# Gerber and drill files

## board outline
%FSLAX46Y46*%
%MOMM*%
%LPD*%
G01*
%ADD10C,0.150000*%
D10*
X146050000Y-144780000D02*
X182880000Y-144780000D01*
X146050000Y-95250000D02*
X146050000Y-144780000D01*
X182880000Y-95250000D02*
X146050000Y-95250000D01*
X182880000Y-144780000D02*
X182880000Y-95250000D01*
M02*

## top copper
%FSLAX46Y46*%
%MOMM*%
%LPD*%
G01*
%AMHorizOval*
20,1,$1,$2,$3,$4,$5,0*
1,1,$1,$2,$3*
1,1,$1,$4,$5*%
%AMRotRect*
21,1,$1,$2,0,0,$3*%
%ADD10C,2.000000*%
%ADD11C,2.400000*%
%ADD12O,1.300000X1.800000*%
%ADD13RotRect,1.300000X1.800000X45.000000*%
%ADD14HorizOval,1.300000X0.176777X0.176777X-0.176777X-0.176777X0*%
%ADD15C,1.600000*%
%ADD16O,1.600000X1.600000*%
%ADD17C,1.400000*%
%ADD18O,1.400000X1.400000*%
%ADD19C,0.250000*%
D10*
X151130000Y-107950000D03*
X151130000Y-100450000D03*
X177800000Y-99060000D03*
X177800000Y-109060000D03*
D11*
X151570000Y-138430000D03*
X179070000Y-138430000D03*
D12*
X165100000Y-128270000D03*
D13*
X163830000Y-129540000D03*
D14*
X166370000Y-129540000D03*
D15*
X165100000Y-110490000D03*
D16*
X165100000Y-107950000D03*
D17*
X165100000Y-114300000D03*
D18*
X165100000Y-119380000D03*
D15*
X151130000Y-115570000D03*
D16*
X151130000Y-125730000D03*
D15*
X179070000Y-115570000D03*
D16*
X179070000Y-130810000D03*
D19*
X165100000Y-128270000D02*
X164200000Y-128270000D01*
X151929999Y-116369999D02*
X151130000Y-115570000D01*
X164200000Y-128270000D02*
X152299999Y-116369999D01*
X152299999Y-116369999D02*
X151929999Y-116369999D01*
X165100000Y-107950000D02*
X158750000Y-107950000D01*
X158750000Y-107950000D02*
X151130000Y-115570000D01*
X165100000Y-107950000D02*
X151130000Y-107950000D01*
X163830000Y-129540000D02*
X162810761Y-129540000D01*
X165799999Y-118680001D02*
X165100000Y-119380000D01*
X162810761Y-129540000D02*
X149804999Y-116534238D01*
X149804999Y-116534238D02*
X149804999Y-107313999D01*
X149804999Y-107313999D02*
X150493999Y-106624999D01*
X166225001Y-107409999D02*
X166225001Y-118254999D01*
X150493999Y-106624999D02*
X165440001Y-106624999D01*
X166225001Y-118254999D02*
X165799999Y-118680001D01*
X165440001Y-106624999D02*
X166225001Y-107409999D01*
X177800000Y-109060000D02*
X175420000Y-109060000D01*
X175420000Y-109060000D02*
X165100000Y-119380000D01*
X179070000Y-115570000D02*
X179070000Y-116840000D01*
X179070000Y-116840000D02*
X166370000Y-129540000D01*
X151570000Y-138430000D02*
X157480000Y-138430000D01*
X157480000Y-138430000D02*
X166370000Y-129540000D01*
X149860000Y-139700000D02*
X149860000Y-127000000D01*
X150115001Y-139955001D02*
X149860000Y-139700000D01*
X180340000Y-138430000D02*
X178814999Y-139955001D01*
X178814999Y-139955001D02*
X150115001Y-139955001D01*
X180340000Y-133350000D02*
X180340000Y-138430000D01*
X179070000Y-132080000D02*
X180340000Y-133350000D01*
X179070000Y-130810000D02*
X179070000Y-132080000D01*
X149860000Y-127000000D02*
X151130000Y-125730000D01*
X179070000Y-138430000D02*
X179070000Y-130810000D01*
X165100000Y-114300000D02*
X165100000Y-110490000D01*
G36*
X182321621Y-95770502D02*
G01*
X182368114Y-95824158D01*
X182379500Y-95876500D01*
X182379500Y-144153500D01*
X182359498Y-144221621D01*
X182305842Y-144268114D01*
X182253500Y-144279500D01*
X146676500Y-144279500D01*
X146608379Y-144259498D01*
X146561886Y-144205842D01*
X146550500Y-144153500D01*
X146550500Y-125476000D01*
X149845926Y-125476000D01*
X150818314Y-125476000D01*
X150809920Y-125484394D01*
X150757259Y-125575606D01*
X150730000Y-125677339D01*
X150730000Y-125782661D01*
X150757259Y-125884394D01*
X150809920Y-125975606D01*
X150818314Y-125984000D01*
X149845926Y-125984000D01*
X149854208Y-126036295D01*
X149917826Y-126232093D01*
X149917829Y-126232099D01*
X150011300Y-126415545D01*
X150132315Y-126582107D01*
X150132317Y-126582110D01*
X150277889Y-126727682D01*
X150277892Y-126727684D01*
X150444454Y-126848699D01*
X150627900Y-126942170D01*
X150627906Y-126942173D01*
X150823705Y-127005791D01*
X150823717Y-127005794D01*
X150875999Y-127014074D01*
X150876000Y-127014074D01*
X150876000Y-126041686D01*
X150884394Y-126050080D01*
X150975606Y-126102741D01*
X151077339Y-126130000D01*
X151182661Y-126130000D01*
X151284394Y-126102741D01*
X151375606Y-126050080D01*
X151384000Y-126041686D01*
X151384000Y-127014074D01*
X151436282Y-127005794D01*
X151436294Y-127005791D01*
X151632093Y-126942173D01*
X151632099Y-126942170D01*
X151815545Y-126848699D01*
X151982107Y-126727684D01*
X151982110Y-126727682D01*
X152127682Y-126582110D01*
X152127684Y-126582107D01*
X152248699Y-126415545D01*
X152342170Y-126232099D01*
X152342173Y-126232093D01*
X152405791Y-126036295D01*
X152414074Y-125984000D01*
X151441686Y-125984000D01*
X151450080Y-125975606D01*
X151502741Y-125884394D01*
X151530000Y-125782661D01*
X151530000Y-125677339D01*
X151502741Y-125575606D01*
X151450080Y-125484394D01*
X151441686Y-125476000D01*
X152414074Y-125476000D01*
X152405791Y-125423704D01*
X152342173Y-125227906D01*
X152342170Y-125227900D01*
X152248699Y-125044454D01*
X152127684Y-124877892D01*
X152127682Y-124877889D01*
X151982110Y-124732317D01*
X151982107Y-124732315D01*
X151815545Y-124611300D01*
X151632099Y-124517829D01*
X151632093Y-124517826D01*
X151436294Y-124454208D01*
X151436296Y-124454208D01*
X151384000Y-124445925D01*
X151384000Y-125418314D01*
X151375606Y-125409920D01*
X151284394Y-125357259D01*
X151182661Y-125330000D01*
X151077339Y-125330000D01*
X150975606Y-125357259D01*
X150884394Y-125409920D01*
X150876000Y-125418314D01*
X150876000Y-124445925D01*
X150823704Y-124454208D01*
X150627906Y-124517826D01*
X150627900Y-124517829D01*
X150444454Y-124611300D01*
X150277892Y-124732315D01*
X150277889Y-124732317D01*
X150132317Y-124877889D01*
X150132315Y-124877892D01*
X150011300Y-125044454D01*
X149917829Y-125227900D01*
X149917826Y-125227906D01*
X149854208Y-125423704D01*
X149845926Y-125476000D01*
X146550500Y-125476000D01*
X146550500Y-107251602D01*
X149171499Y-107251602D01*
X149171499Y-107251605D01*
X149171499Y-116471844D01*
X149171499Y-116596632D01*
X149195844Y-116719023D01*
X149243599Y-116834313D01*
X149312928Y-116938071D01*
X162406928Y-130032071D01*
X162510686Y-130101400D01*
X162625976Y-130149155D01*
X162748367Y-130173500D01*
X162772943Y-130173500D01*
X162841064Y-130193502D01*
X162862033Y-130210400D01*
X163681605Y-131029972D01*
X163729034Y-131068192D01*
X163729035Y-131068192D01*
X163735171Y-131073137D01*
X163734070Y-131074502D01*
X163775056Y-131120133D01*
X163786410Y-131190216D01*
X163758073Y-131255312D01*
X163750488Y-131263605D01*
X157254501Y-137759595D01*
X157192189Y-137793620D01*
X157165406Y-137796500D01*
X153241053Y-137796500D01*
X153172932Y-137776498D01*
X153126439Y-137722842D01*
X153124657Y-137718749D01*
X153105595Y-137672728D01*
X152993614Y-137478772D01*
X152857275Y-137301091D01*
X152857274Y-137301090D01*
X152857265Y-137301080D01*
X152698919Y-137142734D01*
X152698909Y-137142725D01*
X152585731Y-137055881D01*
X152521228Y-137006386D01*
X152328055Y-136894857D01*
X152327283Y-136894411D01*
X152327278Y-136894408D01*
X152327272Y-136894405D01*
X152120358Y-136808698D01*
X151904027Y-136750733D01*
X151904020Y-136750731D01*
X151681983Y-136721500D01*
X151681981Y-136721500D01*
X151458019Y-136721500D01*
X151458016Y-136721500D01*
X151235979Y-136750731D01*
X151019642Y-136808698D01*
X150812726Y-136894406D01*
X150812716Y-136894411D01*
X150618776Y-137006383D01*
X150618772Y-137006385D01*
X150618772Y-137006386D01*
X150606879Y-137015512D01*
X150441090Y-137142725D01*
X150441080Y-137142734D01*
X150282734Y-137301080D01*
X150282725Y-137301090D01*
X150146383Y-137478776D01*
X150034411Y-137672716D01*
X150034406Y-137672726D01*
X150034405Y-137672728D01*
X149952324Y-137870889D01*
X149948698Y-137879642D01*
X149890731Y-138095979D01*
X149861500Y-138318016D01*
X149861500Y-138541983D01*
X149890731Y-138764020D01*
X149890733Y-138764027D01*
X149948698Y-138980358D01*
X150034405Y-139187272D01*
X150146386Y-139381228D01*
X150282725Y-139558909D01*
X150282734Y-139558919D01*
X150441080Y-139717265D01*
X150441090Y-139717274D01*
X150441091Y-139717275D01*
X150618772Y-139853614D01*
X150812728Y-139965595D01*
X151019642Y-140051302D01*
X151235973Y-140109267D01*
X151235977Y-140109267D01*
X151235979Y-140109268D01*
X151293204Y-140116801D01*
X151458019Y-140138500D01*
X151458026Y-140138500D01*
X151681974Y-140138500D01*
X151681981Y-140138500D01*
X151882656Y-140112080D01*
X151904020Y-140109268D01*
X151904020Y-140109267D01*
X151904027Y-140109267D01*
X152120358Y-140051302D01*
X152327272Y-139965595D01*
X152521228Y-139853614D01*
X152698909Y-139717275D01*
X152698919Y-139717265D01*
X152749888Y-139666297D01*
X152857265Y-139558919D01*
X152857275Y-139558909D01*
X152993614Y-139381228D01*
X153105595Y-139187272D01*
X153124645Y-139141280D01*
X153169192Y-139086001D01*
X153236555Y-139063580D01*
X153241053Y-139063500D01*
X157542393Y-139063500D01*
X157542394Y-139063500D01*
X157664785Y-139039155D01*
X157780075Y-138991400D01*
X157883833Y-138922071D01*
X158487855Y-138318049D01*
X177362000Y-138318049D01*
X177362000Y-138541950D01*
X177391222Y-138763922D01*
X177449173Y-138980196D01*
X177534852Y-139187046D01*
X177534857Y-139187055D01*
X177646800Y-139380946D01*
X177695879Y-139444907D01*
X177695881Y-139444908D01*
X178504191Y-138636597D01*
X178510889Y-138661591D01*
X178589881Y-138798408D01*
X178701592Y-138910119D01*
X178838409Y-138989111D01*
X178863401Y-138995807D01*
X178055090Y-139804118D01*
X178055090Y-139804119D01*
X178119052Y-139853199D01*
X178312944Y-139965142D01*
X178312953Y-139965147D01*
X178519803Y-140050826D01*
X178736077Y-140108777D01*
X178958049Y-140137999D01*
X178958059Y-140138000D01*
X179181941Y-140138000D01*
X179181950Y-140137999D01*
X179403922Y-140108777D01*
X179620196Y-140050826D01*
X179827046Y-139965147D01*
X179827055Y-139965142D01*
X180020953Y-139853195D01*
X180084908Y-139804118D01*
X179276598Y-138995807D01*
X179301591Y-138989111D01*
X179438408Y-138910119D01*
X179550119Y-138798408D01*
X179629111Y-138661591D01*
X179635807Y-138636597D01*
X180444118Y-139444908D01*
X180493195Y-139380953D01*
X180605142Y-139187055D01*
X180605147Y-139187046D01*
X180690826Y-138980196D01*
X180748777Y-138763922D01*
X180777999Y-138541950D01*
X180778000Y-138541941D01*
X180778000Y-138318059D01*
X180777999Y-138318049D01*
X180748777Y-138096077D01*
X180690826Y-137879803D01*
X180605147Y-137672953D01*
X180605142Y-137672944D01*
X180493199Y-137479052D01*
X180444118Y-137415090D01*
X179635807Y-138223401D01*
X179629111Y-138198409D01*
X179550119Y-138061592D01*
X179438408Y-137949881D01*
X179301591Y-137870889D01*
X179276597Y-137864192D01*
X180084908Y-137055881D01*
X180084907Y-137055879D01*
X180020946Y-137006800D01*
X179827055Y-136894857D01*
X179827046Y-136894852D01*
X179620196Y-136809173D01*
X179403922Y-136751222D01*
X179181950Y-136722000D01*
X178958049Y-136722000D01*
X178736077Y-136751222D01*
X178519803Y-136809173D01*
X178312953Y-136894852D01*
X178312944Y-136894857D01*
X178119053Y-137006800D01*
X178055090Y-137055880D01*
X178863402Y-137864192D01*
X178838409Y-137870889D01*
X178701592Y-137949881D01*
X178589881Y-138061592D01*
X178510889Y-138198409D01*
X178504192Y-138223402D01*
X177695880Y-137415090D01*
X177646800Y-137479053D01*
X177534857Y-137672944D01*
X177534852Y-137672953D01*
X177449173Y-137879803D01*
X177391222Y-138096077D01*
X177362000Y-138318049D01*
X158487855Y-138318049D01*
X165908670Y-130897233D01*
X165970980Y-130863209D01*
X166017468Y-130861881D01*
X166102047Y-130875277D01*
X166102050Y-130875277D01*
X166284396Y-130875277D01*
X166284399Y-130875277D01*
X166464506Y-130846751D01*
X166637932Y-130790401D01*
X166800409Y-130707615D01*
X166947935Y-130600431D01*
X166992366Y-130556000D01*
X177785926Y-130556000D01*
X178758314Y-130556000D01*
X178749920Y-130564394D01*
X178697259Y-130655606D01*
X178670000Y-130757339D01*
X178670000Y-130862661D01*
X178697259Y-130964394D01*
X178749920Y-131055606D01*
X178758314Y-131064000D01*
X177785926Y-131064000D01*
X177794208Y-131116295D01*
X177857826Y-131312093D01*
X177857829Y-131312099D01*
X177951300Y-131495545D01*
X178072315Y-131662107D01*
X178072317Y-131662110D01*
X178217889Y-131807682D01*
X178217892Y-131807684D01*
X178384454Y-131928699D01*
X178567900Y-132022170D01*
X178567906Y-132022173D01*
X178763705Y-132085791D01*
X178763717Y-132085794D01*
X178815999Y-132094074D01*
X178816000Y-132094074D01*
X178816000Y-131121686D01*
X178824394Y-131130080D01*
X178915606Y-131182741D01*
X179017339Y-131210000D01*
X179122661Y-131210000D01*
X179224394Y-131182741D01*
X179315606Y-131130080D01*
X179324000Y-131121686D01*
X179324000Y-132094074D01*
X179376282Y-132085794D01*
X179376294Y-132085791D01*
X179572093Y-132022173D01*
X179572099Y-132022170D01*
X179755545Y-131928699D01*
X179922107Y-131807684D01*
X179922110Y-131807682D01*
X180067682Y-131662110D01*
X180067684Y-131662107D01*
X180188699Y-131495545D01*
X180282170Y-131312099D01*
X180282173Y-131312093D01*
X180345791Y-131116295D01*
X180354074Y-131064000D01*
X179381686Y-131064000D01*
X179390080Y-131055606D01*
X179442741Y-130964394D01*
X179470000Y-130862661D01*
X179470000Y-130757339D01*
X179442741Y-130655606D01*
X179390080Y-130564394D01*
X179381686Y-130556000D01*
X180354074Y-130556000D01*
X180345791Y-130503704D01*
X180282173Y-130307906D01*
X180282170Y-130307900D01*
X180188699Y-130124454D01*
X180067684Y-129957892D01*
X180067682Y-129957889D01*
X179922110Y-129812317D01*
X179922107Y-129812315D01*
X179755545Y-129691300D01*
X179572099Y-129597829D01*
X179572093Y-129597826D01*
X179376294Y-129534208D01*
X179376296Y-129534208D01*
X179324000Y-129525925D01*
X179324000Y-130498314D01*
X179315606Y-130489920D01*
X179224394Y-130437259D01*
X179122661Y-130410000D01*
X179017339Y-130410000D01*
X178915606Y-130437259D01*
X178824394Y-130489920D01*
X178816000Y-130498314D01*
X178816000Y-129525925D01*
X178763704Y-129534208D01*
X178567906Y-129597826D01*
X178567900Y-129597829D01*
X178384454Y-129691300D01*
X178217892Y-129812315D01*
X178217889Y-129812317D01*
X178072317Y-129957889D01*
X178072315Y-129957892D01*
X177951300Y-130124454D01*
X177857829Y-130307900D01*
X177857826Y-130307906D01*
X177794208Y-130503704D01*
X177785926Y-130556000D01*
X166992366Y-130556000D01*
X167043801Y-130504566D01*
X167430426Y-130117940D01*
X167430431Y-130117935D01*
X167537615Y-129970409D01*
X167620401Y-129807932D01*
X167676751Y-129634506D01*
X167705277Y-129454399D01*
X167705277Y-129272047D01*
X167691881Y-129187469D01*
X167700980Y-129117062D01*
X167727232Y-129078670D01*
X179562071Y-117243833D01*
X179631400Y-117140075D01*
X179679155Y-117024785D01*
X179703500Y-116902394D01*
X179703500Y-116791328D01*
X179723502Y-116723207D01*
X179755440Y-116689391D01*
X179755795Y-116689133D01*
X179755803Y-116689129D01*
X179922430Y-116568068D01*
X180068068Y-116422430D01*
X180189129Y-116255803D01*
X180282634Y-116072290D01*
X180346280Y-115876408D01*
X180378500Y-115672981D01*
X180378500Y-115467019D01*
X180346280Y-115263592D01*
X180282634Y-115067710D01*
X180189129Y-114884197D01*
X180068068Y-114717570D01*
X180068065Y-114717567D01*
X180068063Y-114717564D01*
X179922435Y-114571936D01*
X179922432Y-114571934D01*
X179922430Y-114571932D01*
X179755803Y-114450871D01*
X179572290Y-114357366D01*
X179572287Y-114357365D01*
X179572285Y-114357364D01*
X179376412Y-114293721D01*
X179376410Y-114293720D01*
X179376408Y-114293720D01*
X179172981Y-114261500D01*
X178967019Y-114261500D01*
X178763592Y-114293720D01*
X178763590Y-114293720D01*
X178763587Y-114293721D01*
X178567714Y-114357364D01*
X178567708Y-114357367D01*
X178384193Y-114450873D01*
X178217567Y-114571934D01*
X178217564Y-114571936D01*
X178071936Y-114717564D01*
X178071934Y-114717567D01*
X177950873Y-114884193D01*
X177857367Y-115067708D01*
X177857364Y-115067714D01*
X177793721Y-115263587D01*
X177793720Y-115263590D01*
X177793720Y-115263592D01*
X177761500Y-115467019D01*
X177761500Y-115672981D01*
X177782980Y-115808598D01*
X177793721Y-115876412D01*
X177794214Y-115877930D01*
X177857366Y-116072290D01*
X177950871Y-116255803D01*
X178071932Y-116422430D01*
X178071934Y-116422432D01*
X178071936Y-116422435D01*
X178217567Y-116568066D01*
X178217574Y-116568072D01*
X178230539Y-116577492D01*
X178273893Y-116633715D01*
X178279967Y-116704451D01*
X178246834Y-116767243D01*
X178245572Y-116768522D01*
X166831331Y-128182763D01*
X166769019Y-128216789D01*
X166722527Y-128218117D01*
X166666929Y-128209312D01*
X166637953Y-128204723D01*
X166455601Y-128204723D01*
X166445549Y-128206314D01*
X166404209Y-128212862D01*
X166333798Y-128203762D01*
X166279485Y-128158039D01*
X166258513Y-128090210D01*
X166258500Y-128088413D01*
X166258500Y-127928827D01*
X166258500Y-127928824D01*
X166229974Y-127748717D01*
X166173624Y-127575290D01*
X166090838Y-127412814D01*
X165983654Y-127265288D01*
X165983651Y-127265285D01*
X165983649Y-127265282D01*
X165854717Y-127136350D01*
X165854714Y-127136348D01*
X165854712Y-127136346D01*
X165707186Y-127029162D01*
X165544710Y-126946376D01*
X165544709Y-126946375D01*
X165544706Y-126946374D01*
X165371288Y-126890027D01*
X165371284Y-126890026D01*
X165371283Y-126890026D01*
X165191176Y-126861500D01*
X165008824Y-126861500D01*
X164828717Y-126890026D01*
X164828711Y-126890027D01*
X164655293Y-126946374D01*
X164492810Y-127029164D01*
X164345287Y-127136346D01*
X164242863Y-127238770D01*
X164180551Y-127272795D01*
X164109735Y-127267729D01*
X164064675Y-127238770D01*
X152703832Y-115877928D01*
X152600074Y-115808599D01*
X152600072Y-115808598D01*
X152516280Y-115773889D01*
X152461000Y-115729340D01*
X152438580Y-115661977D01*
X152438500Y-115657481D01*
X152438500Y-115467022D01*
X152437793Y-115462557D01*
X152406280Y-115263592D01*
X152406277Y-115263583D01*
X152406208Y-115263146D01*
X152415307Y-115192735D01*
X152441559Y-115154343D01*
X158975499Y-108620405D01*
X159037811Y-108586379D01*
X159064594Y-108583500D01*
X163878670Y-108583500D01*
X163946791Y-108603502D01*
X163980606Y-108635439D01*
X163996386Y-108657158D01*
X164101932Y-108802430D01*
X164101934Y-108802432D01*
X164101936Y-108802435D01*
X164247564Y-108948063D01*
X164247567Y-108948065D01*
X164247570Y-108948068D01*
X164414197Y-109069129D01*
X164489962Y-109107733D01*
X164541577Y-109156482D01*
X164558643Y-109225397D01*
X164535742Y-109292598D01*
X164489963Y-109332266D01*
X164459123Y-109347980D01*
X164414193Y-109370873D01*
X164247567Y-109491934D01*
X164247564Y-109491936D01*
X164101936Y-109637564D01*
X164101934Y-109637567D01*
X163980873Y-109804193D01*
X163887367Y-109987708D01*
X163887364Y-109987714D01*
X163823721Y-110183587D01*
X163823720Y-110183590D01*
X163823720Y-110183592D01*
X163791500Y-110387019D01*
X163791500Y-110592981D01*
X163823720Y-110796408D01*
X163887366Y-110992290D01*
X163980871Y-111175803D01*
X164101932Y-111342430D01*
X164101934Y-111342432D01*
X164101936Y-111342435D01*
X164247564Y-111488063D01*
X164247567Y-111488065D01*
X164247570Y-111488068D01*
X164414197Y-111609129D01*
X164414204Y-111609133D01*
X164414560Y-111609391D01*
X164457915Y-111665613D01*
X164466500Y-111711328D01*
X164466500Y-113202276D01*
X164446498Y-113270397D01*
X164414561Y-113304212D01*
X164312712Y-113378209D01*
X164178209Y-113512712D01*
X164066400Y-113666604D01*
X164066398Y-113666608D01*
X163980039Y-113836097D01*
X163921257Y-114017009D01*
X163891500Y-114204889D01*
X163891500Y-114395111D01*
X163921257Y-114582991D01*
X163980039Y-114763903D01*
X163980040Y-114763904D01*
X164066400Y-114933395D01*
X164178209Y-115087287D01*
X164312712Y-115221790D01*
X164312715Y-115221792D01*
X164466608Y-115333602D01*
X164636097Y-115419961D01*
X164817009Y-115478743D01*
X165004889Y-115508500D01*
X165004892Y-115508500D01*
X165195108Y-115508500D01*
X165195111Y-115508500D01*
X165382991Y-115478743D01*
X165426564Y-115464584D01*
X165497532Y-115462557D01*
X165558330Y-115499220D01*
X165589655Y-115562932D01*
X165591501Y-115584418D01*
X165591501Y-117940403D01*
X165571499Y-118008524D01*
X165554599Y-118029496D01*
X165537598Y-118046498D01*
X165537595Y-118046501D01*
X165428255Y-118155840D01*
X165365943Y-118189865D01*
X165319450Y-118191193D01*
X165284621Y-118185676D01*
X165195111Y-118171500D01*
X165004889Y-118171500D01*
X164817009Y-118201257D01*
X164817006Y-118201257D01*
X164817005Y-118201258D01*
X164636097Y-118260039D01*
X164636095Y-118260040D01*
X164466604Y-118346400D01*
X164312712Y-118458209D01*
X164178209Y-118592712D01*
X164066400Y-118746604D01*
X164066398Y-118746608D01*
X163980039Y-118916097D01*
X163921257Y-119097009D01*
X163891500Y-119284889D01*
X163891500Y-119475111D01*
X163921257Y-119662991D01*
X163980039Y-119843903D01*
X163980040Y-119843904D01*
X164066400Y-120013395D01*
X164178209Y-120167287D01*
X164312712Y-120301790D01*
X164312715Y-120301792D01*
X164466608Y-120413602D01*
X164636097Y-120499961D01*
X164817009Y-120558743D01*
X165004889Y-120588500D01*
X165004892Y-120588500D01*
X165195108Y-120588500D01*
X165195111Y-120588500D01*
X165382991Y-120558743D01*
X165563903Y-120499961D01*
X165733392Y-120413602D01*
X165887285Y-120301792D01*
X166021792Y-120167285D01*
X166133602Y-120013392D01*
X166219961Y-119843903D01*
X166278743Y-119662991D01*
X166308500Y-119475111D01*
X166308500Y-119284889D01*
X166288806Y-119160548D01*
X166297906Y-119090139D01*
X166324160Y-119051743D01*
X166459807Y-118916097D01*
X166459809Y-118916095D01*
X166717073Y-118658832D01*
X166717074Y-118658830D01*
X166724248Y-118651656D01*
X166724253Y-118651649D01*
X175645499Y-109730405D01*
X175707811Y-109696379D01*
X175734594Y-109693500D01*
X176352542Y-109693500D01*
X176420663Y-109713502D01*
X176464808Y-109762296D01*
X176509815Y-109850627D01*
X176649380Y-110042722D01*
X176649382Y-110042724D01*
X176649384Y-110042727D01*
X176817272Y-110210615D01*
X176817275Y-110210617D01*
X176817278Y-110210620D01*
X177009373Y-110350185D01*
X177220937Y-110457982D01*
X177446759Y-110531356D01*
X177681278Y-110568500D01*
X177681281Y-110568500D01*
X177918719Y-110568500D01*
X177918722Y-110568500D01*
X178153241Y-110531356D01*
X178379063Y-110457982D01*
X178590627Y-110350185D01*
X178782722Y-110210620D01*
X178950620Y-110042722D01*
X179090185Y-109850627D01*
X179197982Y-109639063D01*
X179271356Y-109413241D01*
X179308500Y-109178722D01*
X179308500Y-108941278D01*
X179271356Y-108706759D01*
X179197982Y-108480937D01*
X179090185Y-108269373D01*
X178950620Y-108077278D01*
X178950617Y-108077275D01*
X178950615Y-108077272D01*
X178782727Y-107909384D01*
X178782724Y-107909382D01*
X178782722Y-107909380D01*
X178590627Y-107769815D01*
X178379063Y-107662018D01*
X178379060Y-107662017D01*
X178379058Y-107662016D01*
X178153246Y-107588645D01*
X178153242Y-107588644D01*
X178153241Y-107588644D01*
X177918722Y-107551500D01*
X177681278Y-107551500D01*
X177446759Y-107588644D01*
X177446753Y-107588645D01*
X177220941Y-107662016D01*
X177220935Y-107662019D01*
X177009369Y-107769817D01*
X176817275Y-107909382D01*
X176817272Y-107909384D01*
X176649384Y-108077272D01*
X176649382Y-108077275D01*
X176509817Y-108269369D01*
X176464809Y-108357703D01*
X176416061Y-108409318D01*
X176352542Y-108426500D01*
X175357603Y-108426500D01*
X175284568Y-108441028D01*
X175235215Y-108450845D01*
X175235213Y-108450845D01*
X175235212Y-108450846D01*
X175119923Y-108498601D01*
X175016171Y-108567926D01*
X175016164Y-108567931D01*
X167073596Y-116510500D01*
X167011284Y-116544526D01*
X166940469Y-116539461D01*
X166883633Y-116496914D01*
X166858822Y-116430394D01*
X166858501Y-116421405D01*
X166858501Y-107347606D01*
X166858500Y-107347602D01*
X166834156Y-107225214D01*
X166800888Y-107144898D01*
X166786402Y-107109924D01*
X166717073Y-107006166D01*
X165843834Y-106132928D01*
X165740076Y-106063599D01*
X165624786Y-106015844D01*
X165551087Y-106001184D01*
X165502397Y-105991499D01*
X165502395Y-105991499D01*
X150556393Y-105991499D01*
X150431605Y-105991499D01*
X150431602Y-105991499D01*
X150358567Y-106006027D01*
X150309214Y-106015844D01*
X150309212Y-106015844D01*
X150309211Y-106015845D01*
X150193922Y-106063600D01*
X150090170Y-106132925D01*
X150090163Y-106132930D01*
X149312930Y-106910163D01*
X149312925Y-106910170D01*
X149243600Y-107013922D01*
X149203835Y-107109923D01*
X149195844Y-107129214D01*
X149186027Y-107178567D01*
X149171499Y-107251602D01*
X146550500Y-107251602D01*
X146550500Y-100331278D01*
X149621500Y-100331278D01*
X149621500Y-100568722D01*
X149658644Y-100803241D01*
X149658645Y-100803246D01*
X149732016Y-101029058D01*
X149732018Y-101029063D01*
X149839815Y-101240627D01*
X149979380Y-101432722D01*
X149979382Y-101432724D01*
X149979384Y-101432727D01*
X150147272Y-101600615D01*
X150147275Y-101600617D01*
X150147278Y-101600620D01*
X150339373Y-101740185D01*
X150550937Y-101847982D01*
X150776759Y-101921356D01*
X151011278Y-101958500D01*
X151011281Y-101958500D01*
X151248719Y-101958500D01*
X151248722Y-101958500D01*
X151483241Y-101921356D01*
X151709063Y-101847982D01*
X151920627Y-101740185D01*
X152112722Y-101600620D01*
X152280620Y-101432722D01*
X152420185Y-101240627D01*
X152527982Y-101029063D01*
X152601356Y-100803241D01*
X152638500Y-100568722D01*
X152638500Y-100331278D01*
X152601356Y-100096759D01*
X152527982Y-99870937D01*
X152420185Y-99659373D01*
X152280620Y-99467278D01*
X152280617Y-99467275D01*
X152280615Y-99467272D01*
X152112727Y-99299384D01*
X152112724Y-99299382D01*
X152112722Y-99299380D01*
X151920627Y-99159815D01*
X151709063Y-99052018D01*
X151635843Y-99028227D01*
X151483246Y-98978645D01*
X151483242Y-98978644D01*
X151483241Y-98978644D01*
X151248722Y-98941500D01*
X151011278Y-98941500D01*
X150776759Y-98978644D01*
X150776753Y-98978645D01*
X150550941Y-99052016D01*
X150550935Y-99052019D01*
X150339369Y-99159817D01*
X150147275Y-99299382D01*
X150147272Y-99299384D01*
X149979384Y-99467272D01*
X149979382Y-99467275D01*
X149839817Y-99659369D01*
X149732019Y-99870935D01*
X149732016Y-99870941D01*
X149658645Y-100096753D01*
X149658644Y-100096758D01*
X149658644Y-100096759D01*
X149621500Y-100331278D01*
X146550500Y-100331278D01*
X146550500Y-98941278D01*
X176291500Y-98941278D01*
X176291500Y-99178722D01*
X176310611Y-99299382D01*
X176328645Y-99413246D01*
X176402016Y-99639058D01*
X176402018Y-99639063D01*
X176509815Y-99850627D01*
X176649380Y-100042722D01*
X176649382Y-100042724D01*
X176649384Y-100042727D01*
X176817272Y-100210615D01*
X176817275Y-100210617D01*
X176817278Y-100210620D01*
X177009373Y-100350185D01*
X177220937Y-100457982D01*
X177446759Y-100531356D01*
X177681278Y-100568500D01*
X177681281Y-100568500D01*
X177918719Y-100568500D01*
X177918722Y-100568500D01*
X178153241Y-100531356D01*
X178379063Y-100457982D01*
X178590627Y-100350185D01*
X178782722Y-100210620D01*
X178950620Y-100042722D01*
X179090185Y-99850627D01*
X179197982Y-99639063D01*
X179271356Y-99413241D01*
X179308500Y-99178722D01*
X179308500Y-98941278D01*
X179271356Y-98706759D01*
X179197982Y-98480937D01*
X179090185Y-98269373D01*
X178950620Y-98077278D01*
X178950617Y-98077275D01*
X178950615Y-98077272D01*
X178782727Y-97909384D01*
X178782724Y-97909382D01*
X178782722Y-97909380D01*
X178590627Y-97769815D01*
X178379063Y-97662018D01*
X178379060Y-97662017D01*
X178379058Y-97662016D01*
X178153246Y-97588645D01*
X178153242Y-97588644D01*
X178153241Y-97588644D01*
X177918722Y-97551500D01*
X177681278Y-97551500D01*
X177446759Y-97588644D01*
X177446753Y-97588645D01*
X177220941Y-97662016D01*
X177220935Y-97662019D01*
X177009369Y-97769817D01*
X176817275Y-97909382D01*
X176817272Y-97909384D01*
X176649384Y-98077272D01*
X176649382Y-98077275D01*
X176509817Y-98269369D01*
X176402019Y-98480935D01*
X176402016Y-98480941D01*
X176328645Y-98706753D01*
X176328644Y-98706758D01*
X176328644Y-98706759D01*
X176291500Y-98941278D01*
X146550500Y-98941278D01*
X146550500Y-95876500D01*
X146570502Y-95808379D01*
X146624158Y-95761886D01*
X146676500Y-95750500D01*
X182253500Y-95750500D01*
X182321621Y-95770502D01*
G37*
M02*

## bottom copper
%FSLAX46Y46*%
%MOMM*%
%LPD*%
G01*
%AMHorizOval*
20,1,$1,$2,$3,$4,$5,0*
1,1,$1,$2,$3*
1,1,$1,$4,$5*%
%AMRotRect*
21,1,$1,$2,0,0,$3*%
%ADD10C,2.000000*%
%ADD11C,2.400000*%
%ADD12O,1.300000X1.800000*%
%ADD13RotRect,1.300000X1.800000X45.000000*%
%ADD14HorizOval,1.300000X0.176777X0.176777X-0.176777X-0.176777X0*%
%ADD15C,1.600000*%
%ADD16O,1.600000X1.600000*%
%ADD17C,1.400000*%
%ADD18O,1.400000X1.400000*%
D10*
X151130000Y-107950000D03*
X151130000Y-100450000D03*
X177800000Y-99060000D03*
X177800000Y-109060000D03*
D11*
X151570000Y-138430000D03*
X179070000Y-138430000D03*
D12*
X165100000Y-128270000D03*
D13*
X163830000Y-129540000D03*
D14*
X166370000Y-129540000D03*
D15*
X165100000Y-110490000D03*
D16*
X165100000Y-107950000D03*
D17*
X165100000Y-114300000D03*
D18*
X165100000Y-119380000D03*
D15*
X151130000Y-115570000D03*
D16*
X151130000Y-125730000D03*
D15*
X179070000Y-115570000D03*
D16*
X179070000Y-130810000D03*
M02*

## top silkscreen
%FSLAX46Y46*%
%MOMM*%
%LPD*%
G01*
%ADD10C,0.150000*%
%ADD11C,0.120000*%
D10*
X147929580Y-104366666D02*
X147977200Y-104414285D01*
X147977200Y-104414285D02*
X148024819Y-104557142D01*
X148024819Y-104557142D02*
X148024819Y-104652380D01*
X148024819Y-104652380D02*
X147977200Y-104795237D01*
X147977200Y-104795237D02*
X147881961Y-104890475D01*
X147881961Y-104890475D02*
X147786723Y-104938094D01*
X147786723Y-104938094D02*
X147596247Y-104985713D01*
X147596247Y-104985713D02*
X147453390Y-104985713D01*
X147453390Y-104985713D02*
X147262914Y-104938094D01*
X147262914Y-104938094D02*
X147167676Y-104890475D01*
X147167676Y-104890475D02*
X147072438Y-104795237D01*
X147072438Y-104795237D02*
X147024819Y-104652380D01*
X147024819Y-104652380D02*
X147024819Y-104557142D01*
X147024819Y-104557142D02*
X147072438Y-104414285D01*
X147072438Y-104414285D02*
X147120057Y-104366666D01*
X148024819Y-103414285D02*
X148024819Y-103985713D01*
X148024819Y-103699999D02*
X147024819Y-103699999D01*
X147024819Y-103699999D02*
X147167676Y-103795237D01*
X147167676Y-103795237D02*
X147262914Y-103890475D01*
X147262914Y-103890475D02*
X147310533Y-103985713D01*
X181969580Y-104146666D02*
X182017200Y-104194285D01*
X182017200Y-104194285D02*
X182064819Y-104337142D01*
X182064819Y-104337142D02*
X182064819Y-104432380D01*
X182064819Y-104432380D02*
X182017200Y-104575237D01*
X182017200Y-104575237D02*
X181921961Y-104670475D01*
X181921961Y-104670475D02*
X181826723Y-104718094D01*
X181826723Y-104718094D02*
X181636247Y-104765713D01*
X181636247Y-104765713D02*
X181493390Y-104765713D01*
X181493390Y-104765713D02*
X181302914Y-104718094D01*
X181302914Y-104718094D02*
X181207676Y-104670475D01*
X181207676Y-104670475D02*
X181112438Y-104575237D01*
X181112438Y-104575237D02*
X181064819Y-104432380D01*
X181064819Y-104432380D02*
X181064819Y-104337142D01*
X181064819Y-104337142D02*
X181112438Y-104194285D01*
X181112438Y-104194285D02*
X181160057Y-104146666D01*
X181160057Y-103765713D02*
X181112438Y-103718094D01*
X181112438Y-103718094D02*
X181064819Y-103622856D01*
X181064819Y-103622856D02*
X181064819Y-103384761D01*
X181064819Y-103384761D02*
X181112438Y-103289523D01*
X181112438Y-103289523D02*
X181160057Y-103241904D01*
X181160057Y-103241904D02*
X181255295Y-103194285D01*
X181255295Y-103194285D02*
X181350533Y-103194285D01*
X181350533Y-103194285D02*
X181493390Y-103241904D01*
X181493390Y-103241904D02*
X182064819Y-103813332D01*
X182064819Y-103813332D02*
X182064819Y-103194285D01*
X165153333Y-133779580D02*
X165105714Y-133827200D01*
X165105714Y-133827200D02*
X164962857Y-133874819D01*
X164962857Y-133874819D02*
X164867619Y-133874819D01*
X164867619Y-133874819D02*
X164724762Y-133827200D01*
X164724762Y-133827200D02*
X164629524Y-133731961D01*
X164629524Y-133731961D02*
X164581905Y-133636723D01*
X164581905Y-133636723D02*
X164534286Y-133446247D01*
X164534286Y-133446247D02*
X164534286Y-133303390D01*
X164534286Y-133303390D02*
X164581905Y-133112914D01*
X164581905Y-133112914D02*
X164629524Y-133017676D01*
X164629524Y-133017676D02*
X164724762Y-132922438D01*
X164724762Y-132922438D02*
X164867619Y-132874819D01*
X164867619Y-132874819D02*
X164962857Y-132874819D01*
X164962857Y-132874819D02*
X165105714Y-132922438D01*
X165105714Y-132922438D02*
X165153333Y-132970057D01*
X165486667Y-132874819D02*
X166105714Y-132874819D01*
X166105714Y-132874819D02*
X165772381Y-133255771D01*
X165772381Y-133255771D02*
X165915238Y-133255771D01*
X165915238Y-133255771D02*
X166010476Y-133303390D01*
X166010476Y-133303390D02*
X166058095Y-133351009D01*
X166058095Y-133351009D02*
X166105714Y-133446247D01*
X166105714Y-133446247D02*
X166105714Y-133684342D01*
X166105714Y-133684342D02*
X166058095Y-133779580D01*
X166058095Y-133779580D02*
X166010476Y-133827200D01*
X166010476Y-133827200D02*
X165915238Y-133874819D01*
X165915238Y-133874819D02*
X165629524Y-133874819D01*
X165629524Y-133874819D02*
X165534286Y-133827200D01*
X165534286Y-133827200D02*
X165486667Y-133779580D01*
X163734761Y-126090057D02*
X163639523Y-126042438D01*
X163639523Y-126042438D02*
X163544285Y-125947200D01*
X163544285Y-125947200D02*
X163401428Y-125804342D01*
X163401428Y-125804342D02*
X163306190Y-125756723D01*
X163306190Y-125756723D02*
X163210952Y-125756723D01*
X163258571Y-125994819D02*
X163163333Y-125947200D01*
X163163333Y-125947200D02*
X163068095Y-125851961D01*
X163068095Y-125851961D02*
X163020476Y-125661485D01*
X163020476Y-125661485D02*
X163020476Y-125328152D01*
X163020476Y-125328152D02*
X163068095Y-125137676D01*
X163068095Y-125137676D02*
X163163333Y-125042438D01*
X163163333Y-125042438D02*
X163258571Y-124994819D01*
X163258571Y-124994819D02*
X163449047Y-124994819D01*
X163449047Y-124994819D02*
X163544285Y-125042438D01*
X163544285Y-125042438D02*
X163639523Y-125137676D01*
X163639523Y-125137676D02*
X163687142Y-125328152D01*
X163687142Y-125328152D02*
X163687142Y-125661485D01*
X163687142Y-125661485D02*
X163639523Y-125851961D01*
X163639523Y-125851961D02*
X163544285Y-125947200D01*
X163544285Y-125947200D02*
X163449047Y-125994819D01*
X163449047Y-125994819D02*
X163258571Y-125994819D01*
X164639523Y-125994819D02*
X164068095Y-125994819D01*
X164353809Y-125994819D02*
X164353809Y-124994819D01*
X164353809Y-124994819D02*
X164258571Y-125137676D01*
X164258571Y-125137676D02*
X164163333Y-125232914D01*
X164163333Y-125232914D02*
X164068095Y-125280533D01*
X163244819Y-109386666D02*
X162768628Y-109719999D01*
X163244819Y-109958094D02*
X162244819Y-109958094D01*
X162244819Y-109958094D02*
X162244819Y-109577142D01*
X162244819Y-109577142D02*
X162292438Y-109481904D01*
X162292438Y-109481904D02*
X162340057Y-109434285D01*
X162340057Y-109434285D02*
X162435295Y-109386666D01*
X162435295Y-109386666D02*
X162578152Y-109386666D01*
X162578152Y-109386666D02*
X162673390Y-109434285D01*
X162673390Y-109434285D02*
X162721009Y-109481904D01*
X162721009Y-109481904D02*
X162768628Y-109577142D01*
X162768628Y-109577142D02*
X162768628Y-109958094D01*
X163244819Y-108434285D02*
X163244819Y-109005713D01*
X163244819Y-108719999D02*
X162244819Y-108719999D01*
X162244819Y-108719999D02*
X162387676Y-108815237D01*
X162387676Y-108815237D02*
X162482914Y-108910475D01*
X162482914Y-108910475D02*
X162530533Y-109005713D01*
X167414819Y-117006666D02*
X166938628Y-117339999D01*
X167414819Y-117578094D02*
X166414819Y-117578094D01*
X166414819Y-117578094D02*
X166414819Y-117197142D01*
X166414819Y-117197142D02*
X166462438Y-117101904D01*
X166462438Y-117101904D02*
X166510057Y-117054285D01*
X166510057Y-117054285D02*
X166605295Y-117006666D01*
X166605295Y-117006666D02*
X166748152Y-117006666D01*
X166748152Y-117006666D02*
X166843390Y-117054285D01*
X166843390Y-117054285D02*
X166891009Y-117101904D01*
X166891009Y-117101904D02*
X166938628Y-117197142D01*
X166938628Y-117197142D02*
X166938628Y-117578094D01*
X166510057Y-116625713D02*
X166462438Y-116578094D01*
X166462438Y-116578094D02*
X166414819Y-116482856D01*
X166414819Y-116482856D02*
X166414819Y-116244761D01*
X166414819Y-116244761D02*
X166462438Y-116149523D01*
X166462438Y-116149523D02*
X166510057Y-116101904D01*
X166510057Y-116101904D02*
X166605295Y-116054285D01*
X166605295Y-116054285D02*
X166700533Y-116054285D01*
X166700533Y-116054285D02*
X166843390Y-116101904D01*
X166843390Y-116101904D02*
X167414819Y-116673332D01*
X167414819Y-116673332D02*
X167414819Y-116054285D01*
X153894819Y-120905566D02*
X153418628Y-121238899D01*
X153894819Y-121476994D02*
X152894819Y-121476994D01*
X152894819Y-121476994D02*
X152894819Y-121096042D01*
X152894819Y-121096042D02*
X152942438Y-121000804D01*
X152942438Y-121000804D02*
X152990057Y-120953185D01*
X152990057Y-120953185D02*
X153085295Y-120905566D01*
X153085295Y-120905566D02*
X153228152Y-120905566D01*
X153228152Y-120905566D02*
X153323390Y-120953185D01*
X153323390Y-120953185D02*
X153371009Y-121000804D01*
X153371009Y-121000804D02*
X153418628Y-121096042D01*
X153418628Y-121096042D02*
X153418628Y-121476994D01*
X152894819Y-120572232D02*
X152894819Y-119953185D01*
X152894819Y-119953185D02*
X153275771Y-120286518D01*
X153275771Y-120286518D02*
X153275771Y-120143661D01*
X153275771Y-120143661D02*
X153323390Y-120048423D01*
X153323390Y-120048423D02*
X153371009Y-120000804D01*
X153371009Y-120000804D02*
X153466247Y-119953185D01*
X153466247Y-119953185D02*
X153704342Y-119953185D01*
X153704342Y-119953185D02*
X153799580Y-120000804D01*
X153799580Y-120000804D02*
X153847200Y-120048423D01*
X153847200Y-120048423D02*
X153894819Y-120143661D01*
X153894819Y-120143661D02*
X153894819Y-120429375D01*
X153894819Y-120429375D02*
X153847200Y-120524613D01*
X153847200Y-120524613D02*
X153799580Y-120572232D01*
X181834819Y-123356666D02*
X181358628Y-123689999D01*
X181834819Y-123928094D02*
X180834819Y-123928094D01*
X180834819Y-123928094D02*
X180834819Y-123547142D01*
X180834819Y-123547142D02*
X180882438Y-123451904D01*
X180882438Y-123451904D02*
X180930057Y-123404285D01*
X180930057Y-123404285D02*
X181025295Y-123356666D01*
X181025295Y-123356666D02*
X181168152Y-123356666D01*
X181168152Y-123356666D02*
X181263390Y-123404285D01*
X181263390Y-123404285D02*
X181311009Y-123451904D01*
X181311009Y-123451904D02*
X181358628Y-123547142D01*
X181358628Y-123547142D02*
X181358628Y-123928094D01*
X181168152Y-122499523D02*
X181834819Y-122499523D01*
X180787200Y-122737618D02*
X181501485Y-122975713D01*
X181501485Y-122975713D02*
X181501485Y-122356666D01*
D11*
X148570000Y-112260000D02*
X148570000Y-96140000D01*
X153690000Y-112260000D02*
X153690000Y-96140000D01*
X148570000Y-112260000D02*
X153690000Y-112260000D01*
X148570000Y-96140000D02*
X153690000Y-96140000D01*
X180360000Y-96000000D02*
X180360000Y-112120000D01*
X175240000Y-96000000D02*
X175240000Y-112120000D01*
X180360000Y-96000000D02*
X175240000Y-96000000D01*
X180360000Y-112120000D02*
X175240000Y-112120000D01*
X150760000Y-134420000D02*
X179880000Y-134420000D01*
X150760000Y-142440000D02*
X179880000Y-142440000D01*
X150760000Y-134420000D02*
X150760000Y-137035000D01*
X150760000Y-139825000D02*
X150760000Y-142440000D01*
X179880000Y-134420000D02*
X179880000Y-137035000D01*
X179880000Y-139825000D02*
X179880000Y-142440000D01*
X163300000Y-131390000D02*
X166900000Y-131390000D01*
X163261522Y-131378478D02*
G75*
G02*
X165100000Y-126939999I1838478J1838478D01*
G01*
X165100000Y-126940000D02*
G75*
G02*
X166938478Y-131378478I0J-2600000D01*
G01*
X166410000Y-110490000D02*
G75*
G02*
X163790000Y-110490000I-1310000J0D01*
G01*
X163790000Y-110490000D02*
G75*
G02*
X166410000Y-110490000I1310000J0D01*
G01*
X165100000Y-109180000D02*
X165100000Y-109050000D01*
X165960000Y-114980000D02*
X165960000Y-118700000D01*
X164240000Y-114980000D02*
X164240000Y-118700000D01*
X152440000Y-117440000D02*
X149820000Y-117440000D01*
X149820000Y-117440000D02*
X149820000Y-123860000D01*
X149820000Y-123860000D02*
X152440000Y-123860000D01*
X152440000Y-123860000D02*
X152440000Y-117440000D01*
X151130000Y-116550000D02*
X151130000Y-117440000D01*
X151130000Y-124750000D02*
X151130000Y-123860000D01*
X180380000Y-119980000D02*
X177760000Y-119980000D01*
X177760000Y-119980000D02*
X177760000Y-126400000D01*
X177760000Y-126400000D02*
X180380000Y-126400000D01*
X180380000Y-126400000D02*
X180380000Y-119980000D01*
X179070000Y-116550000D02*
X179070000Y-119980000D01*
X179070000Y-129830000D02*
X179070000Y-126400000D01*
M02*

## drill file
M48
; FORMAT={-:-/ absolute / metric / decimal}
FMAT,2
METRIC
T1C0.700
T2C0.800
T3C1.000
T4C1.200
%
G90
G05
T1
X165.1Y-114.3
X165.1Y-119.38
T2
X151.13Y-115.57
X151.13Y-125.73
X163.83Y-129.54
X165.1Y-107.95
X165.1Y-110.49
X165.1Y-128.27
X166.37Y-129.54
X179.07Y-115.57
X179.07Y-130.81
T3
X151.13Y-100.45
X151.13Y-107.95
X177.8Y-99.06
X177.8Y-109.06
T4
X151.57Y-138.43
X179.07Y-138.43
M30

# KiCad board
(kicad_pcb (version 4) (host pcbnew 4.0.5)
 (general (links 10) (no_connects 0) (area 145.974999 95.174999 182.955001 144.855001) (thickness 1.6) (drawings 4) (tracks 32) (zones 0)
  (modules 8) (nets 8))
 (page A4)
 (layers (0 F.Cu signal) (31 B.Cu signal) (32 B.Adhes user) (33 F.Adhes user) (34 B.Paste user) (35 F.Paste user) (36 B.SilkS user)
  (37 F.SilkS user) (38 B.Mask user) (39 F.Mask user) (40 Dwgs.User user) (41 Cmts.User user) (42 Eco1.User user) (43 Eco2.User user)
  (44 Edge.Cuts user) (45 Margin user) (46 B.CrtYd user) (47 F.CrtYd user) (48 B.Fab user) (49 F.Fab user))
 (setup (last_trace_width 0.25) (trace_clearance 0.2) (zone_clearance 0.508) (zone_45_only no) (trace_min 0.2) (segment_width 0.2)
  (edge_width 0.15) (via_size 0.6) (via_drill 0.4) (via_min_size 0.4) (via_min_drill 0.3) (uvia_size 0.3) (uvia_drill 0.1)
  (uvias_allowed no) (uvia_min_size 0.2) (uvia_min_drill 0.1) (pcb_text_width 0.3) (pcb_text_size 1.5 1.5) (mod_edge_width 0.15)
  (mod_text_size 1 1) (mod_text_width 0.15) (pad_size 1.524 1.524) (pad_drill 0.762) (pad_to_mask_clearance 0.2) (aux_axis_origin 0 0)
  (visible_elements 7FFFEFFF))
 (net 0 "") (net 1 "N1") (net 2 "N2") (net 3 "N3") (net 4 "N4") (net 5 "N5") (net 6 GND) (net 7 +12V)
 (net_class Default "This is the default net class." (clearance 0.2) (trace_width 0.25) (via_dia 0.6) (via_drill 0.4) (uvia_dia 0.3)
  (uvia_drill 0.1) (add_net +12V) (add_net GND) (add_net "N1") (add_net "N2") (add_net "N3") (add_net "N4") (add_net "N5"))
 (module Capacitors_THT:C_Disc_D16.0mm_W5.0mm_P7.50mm (layer F.Cu) (at 151.13 107.95 90)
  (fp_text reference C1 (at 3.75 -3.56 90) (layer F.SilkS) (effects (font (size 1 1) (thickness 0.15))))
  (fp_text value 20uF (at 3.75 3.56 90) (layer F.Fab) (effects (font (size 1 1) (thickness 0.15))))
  (fp_line (start -4.31 -2.56) (end 11.81 -2.56) (layer F.SilkS) (width 0.12))
  (fp_line (start -4.31 2.56) (end 11.81 2.56) (layer F.SilkS) (width 0.12))
  (fp_line (start -4.31 -2.56) (end -4.31 2.56) (layer F.SilkS) (width 0.12))
  (fp_line (start 11.81 -2.56) (end 11.81 2.56) (layer F.SilkS) (width 0.12))
  (pad 1 thru_hole circle (at 0 0 90) (size 2 2) (drill 1) (layers *.Cu *.Mask) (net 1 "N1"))
  (pad 2 thru_hole circle (at 7.5 0 90) (size 2 2) (drill 1) (layers *.Cu *.Mask) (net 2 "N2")))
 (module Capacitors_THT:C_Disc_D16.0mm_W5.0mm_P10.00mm (layer F.Cu) (at 177.8 99.06 270)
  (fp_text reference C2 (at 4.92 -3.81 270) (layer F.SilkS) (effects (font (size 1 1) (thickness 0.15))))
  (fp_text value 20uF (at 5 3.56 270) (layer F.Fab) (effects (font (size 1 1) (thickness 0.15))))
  (fp_line (start -3.06 -2.56) (end 13.06 -2.56) (layer F.SilkS) (width 0.12))
  (fp_line (start -3.06 2.56) (end 13.06 2.56) (layer F.SilkS) (width 0.12))
  (fp_line (start -3.06 -2.56) (end -3.06 2.56) (layer F.SilkS) (width 0.12))
  (fp_line (start 13.06 -2.56) (end 13.06 2.56) (layer F.SilkS) (width 0.12))
  (pad 1 thru_hole circle (at 0 0 270) (size 2 2) (drill 1) (layers *.Cu *.Mask) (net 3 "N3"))
  (pad 2 thru_hole circle (at 10 0 270) (size 2 2) (drill 1) (layers *.Cu *.Mask) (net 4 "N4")))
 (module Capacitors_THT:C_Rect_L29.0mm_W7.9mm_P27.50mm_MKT (layer F.Cu) (at 151.57 138.43)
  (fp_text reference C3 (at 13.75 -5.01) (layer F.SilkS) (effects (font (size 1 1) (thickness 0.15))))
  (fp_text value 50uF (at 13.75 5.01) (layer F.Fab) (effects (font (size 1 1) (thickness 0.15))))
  (fp_line (start -0.81 -4.01) (end 28.31 -4.01) (layer F.SilkS) (width 0.12))
  (fp_line (start -0.81 4.01) (end 28.31 4.01) (layer F.SilkS) (width 0.12))
  (fp_line (start -0.81 -4.01) (end -0.81 -1.395) (layer F.SilkS) (width 0.12))
  (fp_line (start -0.81 1.395) (end -0.81 4.01) (layer F.SilkS) (width 0.12))
  (fp_line (start 28.31 -4.01) (end 28.31 -1.395) (layer F.SilkS) (width 0.12))
  (fp_line (start 28.31 1.395) (end 28.31 4.01) (layer F.SilkS) (width 0.12))
  (pad 1 thru_hole circle (at 0 0) (size 2.4 2.4) (drill 1.2) (layers *.Cu *.Mask) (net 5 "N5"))
  (pad 2 thru_hole circle (at 27.5 0) (size 2.4 2.4) (drill 1.2) (layers *.Cu *.Mask) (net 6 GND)))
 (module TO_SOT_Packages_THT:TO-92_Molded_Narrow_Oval (layer F.Cu) (at 163.83 129.54)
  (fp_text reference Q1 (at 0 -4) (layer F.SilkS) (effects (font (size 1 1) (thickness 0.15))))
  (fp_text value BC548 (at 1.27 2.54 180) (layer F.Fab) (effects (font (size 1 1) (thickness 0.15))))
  (fp_line (start -0.53 1.85) (end 3.07 1.85) (layer F.SilkS) (width 0.12))
  (fp_arc (start 1.27 0) (end 1.27 -2.6) (angle -135) (layer F.SilkS) (width 0.12))
  (fp_arc (start 1.27 0) (end 1.27 -2.6) (angle 135) (layer F.SilkS) (width 0.12))
  (pad 2 thru_hole oval (at 1.27 -1.27 90) (size 1.8 1.3) (drill 0.8) (layers *.Cu *.Mask) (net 1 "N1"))
  (pad 1 thru_hole rect (at 0 0 45) (size 1.3 1.8) (drill 0.8) (layers *.Cu *.Mask) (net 4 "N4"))
  (pad 3 thru_hole oval (at 2.54 0 45) (size 1.8 1.3) (drill 0.8) (layers *.Cu *.Mask) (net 5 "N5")))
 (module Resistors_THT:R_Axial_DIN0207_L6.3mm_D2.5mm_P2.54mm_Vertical (layer F.Cu) (at 165.1 110.49 90)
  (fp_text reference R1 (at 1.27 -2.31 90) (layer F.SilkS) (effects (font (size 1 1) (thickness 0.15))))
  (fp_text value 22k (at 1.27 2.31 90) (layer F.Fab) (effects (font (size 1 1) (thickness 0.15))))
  (fp_circle (center 0 0) (end 1.31 0) (layer F.SilkS) (width 0.12))
  (fp_line (start 1.31 0) (end 1.44 0) (layer F.SilkS) (width 0.12))
  (pad 1 thru_hole circle (at 0 0 90) (size 1.6 1.6) (drill 0.8) (layers *.Cu *.Mask) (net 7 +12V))
  (pad 2 thru_hole oval (at 2.54 0 90) (size 1.6 1.6) (drill 0.8) (layers *.Cu *.Mask) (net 1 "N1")))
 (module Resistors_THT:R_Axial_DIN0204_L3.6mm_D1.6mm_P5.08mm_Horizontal (layer F.Cu) (at 165.1 114.3 270)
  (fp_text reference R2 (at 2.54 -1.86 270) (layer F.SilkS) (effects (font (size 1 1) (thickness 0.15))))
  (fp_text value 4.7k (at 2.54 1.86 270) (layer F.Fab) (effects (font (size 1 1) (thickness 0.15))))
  (fp_line (start 0.68 -0.86) (end 4.4 -0.86) (layer F.SilkS) (width 0.12))
  (fp_line (start 0.68 0.86) (end 4.4 0.86) (layer F.SilkS) (width 0.12))
  (pad 1 thru_hole circle (at 0 0 270) (size 1.4 1.4) (drill 0.7) (layers *.Cu *.Mask) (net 7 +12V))
  (pad 2 thru_hole oval (at 5.08 0 270) (size 1.4 1.4) (drill 0.7) (layers *.Cu *.Mask) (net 4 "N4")))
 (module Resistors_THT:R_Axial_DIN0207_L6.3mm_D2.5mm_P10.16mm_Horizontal (layer F.Cu) (at 151.13 115.57 270)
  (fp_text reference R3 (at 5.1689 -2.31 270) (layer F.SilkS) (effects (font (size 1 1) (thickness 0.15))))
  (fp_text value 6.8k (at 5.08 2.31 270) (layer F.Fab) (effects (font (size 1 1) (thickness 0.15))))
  (fp_line (start 1.87 -1.31) (end 1.87 1.31) (layer F.SilkS) (width 0.12))
  (fp_line (start 1.87 1.31) (end 8.29 1.31) (layer F.SilkS) (width 0.12))
  (fp_line (start 8.29 1.31) (end 8.29 -1.31) (layer F.SilkS) (width 0.12))
  (fp_line (start 8.29 -1.31) (end 1.87 -1.31) (layer F.SilkS) (width 0.12))
  (fp_line (start 0.98 0) (end 1.87 0) (layer F.SilkS) (width 0.12))
  (fp_line (start 9.18 0) (end 8.29 0) (layer F.SilkS) (width 0.12))
  (pad 1 thru_hole circle (at 0 0 270) (size 1.6 1.6) (drill 0.8) (layers *.Cu *.Mask) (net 1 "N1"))
  (pad 2 thru_hole oval (at 10.16 0 270) (size 1.6 1.6) (drill 0.8) (layers *.Cu *.Mask) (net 6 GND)))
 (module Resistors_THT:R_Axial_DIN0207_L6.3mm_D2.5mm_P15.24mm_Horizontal (layer F.Cu) (at 179.07 115.57 270)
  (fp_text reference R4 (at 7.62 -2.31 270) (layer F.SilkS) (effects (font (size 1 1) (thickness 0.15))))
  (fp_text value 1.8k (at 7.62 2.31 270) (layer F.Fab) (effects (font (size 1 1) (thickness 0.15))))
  (fp_line (start 4.41 -1.31) (end 4.41 1.31) (layer F.SilkS) (width 0.12))
  (fp_line (start 4.41 1.31) (end 10.83 1.31) (layer F.SilkS) (width 0.12))
  (fp_line (start 10.83 1.31) (end 10.83 -1.31) (layer F.SilkS) (width 0.12))
  (fp_line (start 10.83 -1.31) (end 4.41 -1.31) (layer F.SilkS) (width 0.12))
  (fp_line (start 0.98 0) (end 4.41 0) (layer F.SilkS) (width 0.12))
  (fp_line (start 14.26 0) (end 10.83 0) (layer F.SilkS) (width 0.12))
  (pad 1 thru_hole circle (at 0 0 270) (size 1.6 1.6) (drill 0.8) (layers *.Cu *.Mask) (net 5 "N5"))
  (pad 2 thru_hole oval (at 15.24 0 270) (size 1.6 1.6) (drill 0.8) (layers *.Cu *.Mask) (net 6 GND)))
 (gr_line (start 146.05 144.78) (end 182.88 144.78) (layer Edge.Cuts) (width 0.15))
 (gr_line (start 146.05 95.25) (end 146.05 144.78) (layer Edge.Cuts) (width 0.15))
 (gr_line (start 182.88 95.25) (end 146.05 95.25) (layer Edge.Cuts) (width 0.15))
 (gr_line (start 182.88 144.78) (end 182.88 95.25) (layer Edge.Cuts) (width 0.15))
 (segment (start 165.1 128.27) (end 164.2 128.27) (width 0.25) (layer F.Cu) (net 1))
 (segment (start 151.929999 116.369999) (end 151.13 115.57) (width 0.25) (layer F.Cu) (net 1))
 (segment (start 164.2 128.27) (end 152.299999 116.369999) (width 0.25) (layer F.Cu) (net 1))
 (segment (start 152.299999 116.369999) (end 151.929999 116.369999) (width 0.25) (layer F.Cu) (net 1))
 (segment (start 165.1 107.95) (end 158.75 107.95) (width 0.25) (layer F.Cu) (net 1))
 (segment (start 158.75 107.95) (end 151.13 115.57) (width 0.25) (layer F.Cu) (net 1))
 (segment (start 165.1 107.95) (end 151.13 107.95) (width 0.25) (layer F.Cu) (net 1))
 (segment (start 163.83 129.54) (end 162.810761 129.54) (width 0.25) (layer F.Cu) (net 4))
 (segment (start 165.799999 118.680001) (end 165.1 119.38) (width 0.25) (layer F.Cu) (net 4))
 (segment (start 162.810761 129.54) (end 149.804999 116.534238) (width 0.25) (layer F.Cu) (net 4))
 (segment (start 149.804999 116.534238) (end 149.804999 107.313999) (width 0.25) (layer F.Cu) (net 4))
 (segment (start 149.804999 107.313999) (end 150.493999 106.624999) (width 0.25) (layer F.Cu) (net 4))
 (segment (start 166.225001 107.409999) (end 166.225001 118.254999) (width 0.25) (layer F.Cu) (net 4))
 (segment (start 150.493999 106.624999) (end 165.440001 106.624999) (width 0.25) (layer F.Cu) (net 4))
 (segment (start 166.225001 118.254999) (end 165.799999 118.680001) (width 0.25) (layer F.Cu) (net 4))
 (segment (start 165.440001 106.624999) (end 166.225001 107.409999) (width 0.25) (layer F.Cu) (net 4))
 (segment (start 177.8 109.06) (end 175.42 109.06) (width 0.25) (layer F.Cu) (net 4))
 (segment (start 175.42 109.06) (end 165.1 119.38) (width 0.25) (layer F.Cu) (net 4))
 (segment (start 179.07 115.57) (end 179.07 116.84) (width 0.25) (layer F.Cu) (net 5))
 (segment (start 179.07 116.84) (end 166.37 129.54) (width 0.25) (layer F.Cu) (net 5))
 (segment (start 151.57 138.43) (end 157.48 138.43) (width 0.25) (layer F.Cu) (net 5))
 (segment (start 157.48 138.43) (end 166.37 129.54) (width 0.25) (layer F.Cu) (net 5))
 (segment (start 149.86 139.7) (end 149.86 127) (width 0.25) (layer F.Cu) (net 6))
 (segment (start 150.115001 139.955001) (end 149.86 139.7) (width 0.25) (layer F.Cu) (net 6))
 (segment (start 180.34 138.43) (end 178.814999 139.955001) (width 0.25) (layer F.Cu) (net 6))
 (segment (start 178.814999 139.955001) (end 150.115001 139.955001) (width 0.25) (layer F.Cu) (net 6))
 (segment (start 180.34 133.35) (end 180.34 138.43) (width 0.25) (layer F.Cu) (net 6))
 (segment (start 179.07 132.08) (end 180.34 133.35) (width 0.25) (layer F.Cu) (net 6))
 (segment (start 179.07 130.81) (end 179.07 132.08) (width 0.25) (layer F.Cu) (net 6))
 (segment (start 149.86 127) (end 151.13 125.73) (width 0.25) (layer F.Cu) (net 6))
 (segment (start 179.07 138.43) (end 179.07 130.81) (width 0.25) (layer F.Cu) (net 6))
 (segment (start 165.1 114.3) (end 165.1 110.49) (width 0.25) (layer F.Cu) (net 7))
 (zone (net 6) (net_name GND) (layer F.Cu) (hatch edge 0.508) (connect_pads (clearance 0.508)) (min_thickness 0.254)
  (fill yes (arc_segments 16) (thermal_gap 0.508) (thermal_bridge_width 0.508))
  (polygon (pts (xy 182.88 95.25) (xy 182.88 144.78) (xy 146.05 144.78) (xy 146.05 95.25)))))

